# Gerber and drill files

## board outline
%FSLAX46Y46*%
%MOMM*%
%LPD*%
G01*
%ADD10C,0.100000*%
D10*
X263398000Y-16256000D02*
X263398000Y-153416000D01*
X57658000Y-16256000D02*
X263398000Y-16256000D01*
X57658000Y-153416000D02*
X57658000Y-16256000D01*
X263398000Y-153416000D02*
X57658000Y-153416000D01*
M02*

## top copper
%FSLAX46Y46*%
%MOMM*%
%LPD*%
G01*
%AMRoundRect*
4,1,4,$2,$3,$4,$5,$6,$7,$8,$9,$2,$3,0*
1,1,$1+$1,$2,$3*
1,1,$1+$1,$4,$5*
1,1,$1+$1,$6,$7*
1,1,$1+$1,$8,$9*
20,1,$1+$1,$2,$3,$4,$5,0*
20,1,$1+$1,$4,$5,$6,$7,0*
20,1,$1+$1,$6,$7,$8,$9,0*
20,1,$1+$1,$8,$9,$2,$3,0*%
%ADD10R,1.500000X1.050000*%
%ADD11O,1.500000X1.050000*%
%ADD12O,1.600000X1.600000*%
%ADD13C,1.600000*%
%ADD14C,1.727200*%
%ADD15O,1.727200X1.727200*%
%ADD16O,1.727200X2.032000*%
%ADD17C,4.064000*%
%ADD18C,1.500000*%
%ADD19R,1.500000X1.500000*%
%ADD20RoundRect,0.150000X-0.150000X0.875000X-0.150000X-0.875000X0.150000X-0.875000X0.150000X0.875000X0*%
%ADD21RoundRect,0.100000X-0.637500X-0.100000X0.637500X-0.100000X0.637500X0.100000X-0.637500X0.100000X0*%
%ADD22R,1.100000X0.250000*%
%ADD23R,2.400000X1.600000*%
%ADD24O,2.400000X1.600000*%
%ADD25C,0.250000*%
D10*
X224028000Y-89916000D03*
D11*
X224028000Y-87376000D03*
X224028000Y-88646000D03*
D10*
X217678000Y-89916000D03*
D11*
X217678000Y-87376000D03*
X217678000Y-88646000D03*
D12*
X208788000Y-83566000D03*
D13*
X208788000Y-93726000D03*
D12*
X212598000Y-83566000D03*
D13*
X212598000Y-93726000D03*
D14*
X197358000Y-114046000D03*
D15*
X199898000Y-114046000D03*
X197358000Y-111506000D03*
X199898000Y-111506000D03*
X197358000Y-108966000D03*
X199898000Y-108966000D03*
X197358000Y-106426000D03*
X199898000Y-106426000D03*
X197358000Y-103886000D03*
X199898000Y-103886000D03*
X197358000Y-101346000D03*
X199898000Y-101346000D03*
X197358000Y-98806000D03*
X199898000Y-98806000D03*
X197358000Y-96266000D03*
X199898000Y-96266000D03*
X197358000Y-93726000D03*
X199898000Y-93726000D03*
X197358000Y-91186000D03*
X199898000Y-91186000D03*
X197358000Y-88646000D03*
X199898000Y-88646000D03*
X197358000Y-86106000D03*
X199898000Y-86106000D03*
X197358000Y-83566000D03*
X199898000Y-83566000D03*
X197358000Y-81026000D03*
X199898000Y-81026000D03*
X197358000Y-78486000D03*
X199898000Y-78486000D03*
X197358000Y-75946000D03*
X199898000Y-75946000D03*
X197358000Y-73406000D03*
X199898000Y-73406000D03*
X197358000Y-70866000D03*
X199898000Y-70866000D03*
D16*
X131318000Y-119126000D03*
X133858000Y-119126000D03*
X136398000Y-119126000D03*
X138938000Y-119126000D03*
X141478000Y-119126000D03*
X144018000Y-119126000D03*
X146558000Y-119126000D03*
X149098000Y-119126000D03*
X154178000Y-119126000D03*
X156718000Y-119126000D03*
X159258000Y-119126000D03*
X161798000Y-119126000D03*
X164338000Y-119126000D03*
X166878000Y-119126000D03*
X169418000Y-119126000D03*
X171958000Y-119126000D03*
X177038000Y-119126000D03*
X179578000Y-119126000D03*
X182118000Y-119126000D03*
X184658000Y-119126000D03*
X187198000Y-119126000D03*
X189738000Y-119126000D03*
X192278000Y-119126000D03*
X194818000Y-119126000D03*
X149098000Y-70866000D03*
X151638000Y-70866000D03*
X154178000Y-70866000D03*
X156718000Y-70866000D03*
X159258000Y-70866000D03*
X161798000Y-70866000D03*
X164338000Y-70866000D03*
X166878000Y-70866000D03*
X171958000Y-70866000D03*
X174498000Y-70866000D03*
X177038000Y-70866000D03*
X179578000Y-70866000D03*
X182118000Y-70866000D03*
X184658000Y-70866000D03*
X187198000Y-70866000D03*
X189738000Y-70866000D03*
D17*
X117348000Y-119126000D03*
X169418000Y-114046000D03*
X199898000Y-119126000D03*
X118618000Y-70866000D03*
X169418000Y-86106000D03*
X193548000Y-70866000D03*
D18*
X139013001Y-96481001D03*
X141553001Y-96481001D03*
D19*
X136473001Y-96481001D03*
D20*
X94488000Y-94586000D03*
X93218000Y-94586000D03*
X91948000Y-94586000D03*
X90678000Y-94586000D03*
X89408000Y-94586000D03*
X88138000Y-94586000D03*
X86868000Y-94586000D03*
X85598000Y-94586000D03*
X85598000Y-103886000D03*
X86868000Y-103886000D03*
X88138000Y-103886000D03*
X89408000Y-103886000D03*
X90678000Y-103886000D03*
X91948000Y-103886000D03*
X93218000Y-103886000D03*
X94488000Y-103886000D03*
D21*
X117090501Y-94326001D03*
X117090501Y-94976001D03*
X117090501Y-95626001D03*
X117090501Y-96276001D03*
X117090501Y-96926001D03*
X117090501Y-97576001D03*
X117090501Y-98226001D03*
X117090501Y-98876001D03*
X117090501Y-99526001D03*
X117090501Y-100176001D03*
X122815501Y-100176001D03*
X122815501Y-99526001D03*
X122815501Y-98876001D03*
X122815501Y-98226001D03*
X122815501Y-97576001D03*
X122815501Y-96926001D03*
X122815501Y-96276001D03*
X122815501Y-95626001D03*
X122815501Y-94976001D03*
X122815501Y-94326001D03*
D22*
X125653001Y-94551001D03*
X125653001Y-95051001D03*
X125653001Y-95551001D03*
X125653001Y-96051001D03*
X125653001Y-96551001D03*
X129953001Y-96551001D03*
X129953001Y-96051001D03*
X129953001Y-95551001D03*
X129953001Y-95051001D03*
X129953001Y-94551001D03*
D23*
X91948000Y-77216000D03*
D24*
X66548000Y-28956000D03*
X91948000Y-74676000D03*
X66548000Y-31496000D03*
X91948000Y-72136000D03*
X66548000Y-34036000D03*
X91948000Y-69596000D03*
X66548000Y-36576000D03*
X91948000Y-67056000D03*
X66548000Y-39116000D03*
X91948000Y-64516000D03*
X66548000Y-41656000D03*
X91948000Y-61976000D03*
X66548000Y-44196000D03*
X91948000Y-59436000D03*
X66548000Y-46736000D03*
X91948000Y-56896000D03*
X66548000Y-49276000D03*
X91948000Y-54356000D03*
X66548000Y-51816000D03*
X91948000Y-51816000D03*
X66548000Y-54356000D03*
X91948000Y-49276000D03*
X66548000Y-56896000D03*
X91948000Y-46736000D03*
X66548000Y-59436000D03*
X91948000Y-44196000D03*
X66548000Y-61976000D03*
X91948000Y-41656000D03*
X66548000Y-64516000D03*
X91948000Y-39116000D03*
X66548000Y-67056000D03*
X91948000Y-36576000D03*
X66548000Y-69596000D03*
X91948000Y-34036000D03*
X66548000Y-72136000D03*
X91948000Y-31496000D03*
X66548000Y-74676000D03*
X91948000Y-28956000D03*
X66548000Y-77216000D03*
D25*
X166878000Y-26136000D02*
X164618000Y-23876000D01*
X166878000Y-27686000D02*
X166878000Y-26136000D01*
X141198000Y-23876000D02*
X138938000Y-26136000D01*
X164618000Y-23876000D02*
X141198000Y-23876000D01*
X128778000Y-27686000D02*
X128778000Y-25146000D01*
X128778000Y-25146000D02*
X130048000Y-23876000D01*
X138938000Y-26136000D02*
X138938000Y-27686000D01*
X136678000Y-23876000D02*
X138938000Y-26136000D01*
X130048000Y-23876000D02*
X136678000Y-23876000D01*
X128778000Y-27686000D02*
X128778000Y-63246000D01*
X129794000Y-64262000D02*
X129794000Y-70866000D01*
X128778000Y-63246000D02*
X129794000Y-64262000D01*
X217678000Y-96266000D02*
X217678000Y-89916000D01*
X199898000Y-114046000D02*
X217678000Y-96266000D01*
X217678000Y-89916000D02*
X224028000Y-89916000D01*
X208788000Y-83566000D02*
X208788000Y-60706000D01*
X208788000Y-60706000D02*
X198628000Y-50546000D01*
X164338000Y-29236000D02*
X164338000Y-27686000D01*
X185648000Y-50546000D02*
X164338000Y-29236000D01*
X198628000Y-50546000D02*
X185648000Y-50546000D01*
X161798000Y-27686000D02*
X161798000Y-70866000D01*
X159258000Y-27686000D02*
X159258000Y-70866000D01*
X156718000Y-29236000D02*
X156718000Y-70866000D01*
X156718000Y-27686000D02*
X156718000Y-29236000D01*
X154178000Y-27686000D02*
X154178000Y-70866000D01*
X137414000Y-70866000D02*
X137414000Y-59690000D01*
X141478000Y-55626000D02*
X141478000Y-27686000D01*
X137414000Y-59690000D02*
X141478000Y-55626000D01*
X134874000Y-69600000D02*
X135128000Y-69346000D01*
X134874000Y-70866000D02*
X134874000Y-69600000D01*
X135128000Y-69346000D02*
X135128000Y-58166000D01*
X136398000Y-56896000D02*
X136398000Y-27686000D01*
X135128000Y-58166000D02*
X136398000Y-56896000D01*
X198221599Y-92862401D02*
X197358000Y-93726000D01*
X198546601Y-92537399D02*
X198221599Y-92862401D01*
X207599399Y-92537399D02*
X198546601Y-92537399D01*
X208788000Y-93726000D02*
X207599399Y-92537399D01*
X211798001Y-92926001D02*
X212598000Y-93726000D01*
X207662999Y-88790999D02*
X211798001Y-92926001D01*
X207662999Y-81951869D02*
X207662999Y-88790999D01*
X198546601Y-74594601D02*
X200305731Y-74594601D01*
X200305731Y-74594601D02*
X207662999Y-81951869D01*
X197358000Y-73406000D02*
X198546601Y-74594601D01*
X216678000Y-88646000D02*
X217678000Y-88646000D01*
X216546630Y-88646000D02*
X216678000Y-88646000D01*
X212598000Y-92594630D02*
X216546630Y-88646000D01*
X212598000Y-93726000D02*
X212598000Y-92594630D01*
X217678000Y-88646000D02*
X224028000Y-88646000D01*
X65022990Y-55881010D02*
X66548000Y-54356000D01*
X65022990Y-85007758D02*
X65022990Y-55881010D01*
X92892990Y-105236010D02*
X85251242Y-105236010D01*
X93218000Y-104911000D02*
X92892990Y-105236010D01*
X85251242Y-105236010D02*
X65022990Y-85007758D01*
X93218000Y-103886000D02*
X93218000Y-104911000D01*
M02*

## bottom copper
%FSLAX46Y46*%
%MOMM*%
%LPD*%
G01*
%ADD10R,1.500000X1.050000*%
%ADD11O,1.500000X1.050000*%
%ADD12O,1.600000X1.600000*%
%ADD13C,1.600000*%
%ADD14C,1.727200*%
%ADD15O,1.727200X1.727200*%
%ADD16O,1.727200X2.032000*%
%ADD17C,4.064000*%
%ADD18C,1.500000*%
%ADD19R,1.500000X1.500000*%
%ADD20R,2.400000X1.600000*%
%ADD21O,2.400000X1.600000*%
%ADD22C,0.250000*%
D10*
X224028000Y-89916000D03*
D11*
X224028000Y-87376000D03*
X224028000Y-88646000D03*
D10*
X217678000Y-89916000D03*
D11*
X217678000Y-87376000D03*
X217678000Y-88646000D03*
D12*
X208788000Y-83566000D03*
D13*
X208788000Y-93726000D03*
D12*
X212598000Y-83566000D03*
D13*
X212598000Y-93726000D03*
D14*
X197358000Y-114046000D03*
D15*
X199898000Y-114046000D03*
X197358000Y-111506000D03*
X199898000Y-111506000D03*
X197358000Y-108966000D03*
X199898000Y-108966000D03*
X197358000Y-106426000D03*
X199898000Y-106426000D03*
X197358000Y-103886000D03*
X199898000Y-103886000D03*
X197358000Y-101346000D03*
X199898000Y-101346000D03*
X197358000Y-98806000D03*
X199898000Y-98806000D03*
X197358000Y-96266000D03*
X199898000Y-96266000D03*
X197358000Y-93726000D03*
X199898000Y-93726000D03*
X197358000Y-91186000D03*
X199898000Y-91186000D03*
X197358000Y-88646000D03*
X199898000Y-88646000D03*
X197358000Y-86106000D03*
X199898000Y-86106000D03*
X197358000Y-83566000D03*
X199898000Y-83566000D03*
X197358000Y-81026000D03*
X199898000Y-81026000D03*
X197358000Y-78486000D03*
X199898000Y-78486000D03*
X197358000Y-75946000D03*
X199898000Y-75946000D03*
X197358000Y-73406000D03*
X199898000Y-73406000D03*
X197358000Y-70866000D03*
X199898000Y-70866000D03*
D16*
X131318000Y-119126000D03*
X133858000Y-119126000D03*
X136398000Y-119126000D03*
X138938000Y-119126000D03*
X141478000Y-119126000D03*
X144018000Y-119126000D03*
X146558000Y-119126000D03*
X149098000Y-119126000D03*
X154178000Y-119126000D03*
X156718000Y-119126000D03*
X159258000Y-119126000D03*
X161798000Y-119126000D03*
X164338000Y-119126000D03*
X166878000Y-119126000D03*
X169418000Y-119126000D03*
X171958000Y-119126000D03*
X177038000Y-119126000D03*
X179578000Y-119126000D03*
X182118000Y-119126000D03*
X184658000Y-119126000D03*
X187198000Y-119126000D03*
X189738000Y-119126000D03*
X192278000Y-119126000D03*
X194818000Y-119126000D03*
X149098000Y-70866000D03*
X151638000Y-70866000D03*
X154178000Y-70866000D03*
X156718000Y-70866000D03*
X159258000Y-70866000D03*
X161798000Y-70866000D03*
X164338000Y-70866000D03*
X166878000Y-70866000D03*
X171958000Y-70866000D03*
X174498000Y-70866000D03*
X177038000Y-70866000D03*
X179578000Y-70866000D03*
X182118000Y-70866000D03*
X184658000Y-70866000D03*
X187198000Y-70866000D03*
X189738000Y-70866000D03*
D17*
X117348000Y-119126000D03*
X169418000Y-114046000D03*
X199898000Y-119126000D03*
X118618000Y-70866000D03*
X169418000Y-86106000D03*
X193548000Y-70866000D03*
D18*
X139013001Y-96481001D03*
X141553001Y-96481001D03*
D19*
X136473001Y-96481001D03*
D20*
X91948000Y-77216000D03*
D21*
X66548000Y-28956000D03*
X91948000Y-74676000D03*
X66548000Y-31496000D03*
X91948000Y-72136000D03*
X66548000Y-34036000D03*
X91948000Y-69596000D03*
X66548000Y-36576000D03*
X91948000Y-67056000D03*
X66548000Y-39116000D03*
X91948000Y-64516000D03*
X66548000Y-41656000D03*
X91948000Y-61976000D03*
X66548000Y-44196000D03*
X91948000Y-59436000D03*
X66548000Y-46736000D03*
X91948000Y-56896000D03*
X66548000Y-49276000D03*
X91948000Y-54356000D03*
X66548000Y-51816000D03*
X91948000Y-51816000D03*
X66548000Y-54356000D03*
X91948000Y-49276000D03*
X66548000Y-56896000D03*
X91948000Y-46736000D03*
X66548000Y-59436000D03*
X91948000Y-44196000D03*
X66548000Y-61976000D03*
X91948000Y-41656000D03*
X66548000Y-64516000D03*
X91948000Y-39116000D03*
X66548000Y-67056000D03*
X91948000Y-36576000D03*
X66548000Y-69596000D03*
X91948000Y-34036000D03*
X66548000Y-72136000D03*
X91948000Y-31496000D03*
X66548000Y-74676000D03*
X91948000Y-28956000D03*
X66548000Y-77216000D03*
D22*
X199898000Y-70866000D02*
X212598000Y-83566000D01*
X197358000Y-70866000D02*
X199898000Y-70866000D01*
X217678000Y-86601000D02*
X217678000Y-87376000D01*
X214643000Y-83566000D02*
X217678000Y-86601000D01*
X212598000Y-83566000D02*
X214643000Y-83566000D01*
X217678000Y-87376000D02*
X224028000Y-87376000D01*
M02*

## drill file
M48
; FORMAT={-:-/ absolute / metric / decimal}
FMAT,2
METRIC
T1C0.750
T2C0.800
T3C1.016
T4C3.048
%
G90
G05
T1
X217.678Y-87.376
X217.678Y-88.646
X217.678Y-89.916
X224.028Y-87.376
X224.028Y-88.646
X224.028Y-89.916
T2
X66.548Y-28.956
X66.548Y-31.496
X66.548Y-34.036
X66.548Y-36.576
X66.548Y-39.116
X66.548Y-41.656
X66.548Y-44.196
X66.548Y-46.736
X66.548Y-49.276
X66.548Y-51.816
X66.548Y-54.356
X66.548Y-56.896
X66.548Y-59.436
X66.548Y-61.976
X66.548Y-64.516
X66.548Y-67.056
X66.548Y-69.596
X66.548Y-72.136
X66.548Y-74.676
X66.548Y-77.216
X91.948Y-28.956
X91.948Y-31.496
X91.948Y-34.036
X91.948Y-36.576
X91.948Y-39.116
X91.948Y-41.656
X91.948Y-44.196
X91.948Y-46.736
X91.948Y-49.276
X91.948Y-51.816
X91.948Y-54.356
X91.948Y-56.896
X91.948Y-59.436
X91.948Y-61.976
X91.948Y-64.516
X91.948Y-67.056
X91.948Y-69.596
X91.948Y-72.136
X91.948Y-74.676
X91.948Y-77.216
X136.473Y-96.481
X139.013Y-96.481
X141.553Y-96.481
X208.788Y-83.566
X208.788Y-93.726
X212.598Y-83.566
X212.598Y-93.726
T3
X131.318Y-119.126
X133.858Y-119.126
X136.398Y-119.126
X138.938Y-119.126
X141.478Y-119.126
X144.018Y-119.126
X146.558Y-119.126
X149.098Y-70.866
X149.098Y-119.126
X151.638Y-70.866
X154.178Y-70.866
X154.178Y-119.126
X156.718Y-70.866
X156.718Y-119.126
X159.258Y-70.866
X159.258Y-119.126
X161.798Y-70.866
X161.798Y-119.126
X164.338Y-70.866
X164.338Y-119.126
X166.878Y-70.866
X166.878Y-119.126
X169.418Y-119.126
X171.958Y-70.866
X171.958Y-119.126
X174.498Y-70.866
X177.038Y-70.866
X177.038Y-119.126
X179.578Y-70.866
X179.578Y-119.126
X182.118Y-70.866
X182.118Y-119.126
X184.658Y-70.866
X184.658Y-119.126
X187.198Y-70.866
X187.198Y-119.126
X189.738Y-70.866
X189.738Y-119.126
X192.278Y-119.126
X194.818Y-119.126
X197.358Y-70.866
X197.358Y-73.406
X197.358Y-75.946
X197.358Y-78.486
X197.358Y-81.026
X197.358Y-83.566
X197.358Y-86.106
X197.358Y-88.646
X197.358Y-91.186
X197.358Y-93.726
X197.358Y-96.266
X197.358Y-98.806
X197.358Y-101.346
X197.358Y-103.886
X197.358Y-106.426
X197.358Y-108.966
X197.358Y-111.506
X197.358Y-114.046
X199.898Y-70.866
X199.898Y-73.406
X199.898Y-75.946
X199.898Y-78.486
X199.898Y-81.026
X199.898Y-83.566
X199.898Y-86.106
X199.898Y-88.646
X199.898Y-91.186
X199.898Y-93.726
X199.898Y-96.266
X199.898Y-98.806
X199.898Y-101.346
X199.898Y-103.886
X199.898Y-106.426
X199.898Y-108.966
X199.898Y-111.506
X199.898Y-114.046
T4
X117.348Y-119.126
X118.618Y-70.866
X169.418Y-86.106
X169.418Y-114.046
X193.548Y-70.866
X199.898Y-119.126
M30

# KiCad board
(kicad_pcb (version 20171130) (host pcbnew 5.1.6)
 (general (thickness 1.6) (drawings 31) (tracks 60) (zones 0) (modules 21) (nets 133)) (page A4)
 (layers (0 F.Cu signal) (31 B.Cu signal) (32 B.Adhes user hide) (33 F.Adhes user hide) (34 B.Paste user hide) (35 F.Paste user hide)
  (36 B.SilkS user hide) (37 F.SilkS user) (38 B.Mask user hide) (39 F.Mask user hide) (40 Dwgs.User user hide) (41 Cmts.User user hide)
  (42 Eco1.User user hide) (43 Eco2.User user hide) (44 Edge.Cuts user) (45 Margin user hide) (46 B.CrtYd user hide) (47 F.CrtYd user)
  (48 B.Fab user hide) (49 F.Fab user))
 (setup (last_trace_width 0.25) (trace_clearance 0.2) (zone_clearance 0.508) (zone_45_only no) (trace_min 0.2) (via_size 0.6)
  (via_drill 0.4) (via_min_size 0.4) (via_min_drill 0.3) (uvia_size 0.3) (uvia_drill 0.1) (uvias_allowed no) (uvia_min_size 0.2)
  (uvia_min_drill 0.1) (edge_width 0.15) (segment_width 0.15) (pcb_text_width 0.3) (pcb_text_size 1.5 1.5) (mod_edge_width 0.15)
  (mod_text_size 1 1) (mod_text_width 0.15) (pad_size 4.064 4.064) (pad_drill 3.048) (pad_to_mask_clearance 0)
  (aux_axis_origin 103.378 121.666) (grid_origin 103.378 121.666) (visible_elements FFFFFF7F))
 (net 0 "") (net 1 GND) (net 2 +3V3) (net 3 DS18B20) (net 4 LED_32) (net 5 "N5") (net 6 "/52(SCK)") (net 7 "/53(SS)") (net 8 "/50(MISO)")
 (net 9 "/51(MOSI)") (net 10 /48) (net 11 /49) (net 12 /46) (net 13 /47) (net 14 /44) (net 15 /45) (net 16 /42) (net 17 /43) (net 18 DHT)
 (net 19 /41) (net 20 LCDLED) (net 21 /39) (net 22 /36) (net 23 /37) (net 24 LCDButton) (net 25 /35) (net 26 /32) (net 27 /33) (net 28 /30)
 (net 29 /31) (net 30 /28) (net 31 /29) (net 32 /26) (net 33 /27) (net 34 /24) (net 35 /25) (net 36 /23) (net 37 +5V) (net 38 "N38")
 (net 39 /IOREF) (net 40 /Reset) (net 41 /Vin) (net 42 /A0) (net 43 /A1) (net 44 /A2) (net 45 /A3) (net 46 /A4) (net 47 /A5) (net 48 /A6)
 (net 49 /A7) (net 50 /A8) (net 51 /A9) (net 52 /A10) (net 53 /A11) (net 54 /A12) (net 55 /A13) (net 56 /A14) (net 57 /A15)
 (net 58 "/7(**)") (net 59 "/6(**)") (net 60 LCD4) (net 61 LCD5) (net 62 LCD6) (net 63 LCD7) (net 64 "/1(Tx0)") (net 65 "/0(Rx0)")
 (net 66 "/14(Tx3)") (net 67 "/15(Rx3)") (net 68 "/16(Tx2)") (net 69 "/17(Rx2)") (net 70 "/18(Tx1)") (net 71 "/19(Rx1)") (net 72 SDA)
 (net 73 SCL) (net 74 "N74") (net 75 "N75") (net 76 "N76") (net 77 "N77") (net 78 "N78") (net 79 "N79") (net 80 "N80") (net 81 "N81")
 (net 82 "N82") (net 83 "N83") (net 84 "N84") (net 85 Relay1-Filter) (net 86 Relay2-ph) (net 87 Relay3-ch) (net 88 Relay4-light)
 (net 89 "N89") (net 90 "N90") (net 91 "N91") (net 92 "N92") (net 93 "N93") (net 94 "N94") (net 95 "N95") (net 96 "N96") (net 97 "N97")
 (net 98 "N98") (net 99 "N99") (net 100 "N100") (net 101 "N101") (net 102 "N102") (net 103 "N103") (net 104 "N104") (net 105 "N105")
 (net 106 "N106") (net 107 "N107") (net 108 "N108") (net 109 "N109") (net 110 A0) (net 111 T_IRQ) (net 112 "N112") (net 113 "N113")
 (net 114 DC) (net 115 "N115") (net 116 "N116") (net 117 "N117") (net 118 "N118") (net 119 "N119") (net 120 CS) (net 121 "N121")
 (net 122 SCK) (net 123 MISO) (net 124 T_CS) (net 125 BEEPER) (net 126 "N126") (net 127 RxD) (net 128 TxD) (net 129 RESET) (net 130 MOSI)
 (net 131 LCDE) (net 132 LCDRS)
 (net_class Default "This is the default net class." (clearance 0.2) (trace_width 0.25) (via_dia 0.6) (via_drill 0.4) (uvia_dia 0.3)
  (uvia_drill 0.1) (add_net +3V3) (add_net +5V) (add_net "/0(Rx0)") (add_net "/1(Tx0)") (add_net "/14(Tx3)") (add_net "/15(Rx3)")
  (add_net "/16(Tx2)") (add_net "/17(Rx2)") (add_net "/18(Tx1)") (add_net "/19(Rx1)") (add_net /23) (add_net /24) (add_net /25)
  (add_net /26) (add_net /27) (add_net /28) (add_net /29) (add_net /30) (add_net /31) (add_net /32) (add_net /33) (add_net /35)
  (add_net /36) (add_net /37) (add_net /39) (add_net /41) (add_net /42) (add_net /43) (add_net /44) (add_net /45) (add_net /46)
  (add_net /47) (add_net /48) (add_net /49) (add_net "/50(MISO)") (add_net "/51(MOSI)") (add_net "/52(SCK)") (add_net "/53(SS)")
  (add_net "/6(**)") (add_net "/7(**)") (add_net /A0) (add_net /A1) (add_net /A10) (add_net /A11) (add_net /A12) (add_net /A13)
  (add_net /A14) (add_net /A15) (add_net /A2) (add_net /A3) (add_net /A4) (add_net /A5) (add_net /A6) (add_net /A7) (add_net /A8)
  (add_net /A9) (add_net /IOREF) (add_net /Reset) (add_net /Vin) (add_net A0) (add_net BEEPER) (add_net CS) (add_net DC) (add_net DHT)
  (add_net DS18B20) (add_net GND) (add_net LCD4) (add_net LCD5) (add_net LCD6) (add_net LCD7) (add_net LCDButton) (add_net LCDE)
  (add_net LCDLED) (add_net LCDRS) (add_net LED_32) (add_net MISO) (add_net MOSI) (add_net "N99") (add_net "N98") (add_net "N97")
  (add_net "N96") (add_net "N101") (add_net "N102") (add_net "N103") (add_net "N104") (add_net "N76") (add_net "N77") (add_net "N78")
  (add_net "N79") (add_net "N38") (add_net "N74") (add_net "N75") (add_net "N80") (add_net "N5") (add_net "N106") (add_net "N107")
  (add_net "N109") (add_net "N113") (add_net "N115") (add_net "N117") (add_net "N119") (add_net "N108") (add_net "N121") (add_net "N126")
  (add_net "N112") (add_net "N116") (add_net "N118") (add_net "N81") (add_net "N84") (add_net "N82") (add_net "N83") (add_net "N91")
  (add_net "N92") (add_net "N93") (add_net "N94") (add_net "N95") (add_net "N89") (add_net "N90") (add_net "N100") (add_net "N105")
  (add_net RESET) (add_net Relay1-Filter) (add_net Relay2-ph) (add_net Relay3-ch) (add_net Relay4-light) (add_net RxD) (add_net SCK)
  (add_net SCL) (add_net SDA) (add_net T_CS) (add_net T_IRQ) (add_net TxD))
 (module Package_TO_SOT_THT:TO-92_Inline (layer F.Cu) (at 224.028 89.916 90)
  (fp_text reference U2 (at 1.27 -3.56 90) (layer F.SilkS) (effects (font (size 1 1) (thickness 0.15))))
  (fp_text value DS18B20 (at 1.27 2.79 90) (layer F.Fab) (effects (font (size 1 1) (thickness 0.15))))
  (pad 1 thru_hole rect (at 0 0 90) (size 1.05 1.5) (drill 0.75) (layers *.Cu *.Mask) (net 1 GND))
  (pad 3 thru_hole oval (at 2.54 0 90) (size 1.05 1.5) (drill 0.75) (layers *.Cu *.Mask) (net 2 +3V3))
  (pad 2 thru_hole oval (at 1.27 0 90) (size 1.05 1.5) (drill 0.75) (layers *.Cu *.Mask) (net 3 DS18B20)))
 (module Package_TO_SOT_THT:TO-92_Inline (layer F.Cu) (at 217.678 89.916 90)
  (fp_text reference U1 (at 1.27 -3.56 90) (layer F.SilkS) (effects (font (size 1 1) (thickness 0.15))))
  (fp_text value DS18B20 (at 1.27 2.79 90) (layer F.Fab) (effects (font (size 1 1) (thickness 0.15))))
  (pad 1 thru_hole rect (at 0 0 90) (size 1.05 1.5) (drill 0.75) (layers *.Cu *.Mask) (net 1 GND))
  (pad 3 thru_hole oval (at 2.54 0 90) (size 1.05 1.5) (drill 0.75) (layers *.Cu *.Mask) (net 2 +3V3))
  (pad 2 thru_hole oval (at 1.27 0 90) (size 1.05 1.5) (drill 0.75) (layers *.Cu *.Mask) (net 3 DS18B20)))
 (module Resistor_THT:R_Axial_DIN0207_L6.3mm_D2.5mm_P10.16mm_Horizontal (layer F.Cu) (at 208.788 93.726 90)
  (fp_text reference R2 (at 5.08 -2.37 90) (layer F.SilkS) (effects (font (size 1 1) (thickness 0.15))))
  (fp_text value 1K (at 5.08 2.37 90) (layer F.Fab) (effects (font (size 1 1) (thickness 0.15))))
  (pad 2 thru_hole oval (at 10.16 0 90) (size 1.6 1.6) (drill 0.8) (layers *.Cu *.Mask) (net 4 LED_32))
  (pad 1 thru_hole circle (at 0 0 90) (size 1.6 1.6) (drill 0.8) (layers *.Cu *.Mask) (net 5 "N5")))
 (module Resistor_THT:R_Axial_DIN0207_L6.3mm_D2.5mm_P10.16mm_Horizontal (layer F.Cu) (at 212.598 93.726 90)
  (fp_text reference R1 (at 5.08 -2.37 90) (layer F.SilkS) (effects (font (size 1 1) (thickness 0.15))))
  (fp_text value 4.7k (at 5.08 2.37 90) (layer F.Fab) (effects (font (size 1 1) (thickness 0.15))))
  (pad 2 thru_hole oval (at 10.16 0 90) (size 1.6 1.6) (drill 0.8) (layers *.Cu *.Mask) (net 2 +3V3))
  (pad 1 thru_hole circle (at 0 0 90) (size 1.6 1.6) (drill 0.8) (layers *.Cu *.Mask) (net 3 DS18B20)))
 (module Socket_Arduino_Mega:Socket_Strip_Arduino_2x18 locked (layer F.Cu) (at 197.358 114.046 90)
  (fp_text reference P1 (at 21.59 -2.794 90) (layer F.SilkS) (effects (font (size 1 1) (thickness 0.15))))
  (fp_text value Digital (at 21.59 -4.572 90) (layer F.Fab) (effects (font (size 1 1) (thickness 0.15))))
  (pad 1 thru_hole circle (at 0 0 90) (size 1.7272 1.7272) (drill 1.016) (layers *.Cu *.Mask F.SilkS) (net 1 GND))
  (pad 2 thru_hole oval (at 0 2.54 90) (size 1.7272 1.7272) (drill 1.016) (layers *.Cu *.Mask F.SilkS) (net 1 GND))
  (pad 3 thru_hole oval (at 2.54 0 90) (size 1.7272 1.7272) (drill 1.016) (layers *.Cu *.Mask F.SilkS) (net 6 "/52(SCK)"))
  (pad 4 thru_hole oval (at 2.54 2.54 90) (size 1.7272 1.7272) (drill 1.016) (layers *.Cu *.Mask F.SilkS) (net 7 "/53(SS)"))
  (pad 5 thru_hole oval (at 5.08 0 90) (size 1.7272 1.7272) (drill 1.016) (layers *.Cu *.Mask F.SilkS) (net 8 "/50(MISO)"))
  (pad 6 thru_hole oval (at 5.08 2.54 90) (size 1.7272 1.7272) (drill 1.016) (layers *.Cu *.Mask F.SilkS) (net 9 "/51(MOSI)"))
  (pad 7 thru_hole oval (at 7.62 0 90) (size 1.7272 1.7272) (drill 1.016) (layers *.Cu *.Mask F.SilkS) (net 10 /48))
  (pad 8 thru_hole oval (at 7.62 2.54 90) (size 1.7272 1.7272) (drill 1.016) (layers *.Cu *.Mask F.SilkS) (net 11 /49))
  (pad 9 thru_hole oval (at 10.16 0 90) (size 1.7272 1.7272) (drill 1.016) (layers *.Cu *.Mask F.SilkS) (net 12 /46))
  (pad 10 thru_hole oval (at 10.16 2.54 90) (size 1.7272 1.7272) (drill 1.016) (layers *.Cu *.Mask F.SilkS) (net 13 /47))
  (pad 11 thru_hole oval (at 12.7 0 90) (size 1.7272 1.7272) (drill 1.016) (layers *.Cu *.Mask F.SilkS) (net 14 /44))
  (pad 12 thru_hole oval (at 12.7 2.54 90) (size 1.7272 1.7272) (drill 1.016) (layers *.Cu *.Mask F.SilkS) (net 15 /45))
  (pad 13 thru_hole oval (at 15.24 0 90) (size 1.7272 1.7272) (drill 1.016) (layers *.Cu *.Mask F.SilkS) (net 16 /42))
  (pad 14 thru_hole oval (at 15.24 2.54 90) (size 1.7272 1.7272) (drill 1.016) (layers *.Cu *.Mask F.SilkS) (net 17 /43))
  (pad 15 thru_hole oval (at 17.78 0 90) (size 1.7272 1.7272) (drill 1.016) (layers *.Cu *.Mask F.SilkS) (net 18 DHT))
  (pad 16 thru_hole oval (at 17.78 2.54 90) (size 1.7272 1.7272) (drill 1.016) (layers *.Cu *.Mask F.SilkS) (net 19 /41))
  (pad 17 thru_hole oval (at 20.32 0 90) (size 1.7272 1.7272) (drill 1.016) (layers *.Cu *.Mask F.SilkS) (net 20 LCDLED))
  (pad 18 thru_hole oval (at 20.32 2.54 90) (size 1.7272 1.7272) (drill 1.016) (layers *.Cu *.Mask F.SilkS) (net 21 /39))
  (pad 19 thru_hole oval (at 22.86 0 90) (size 1.7272 1.7272) (drill 1.016) (layers *.Cu *.Mask F.SilkS) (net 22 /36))
  (pad 20 thru_hole oval (at 22.86 2.54 90) (size 1.7272 1.7272) (drill 1.016) (layers *.Cu *.Mask F.SilkS) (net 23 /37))
  (pad 21 thru_hole oval (at 25.4 0 90) (size 1.7272 1.7272) (drill 1.016) (layers *.Cu *.Mask F.SilkS) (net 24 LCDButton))
  (pad 22 thru_hole oval (at 25.4 2.54 90) (size 1.7272 1.7272) (drill 1.016) (layers *.Cu *.Mask F.SilkS) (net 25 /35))
  (pad 23 thru_hole oval (at 27.94 0 90) (size 1.7272 1.7272) (drill 1.016) (layers *.Cu *.Mask F.SilkS) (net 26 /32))
  (pad 24 thru_hole oval (at 27.94 2.54 90) (size 1.7272 1.7272) (drill 1.016) (layers *.Cu *.Mask F.SilkS) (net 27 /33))
  (pad 25 thru_hole oval (at 30.48 0 90) (size 1.7272 1.7272) (drill 1.016) (layers *.Cu *.Mask F.SilkS) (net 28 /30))
  (pad 26 thru_hole oval (at 30.48 2.54 90) (size 1.7272 1.7272) (drill 1.016) (layers *.Cu *.Mask F.SilkS) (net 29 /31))
  (pad 27 thru_hole oval (at 33.02 0 90) (size 1.7272 1.7272) (drill 1.016) (layers *.Cu *.Mask F.SilkS) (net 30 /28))
  (pad 28 thru_hole oval (at 33.02 2.54 90) (size 1.7272 1.7272) (drill 1.016) (layers *.Cu *.Mask F.SilkS) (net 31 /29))
  (pad 29 thru_hole oval (at 35.56 0 90) (size 1.7272 1.7272) (drill 1.016) (layers *.Cu *.Mask F.SilkS) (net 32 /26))
  (pad 30 thru_hole oval (at 35.56 2.54 90) (size 1.7272 1.7272) (drill 1.016) (layers *.Cu *.Mask F.SilkS) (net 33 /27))
  (pad 31 thru_hole oval (at 38.1 0 90) (size 1.7272 1.7272) (drill 1.016) (layers *.Cu *.Mask F.SilkS) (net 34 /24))
  (pad 32 thru_hole oval (at 38.1 2.54 90) (size 1.7272 1.7272) (drill 1.016) (layers *.Cu *.Mask F.SilkS) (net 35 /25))
  (pad 33 thru_hole oval (at 40.64 0 90) (size 1.7272 1.7272) (drill 1.016) (layers *.Cu *.Mask F.SilkS) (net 3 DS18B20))
  (pad 34 thru_hole oval (at 40.64 2.54 90) (size 1.7272 1.7272) (drill 1.016) (layers *.Cu *.Mask F.SilkS) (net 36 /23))
  (pad 35 thru_hole oval (at 43.18 0 90) (size 1.7272 1.7272) (drill 1.016) (layers *.Cu *.Mask F.SilkS) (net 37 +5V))
  (pad 36 thru_hole oval (at 43.18 2.54 90) (size 1.7272 1.7272) (drill 1.016) (layers *.Cu *.Mask F.SilkS) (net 37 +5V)))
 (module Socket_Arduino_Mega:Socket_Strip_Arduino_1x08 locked (layer F.Cu) (at 131.318 119.126)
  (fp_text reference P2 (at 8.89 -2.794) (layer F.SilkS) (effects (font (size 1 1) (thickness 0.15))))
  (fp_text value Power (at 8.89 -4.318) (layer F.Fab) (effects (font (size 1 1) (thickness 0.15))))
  (pad 1 thru_hole oval (at 0 0) (size 1.7272 2.032) (drill 1.016) (layers *.Cu *.Mask F.SilkS) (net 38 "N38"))
  (pad 2 thru_hole oval (at 2.54 0) (size 1.7272 2.032) (drill 1.016) (layers *.Cu *.Mask F.SilkS) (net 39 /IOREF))
  (pad 3 thru_hole oval (at 5.08 0) (size 1.7272 2.032) (drill 1.016) (layers *.Cu *.Mask F.SilkS) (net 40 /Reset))
  (pad 4 thru_hole oval (at 7.62 0) (size 1.7272 2.032) (drill 1.016) (layers *.Cu *.Mask F.SilkS) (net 2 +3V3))
  (pad 5 thru_hole oval (at 10.16 0) (size 1.7272 2.032) (drill 1.016) (layers *.Cu *.Mask F.SilkS) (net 37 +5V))
  (pad 6 thru_hole oval (at 12.7 0) (size 1.7272 2.032) (drill 1.016) (layers *.Cu *.Mask F.SilkS) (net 1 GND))
  (pad 7 thru_hole oval (at 15.24 0) (size 1.7272 2.032) (drill 1.016) (layers *.Cu *.Mask F.SilkS) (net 1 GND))
  (pad 8 thru_hole oval (at 17.78 0) (size 1.7272 2.032) (drill 1.016) (layers *.Cu *.Mask F.SilkS) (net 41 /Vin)))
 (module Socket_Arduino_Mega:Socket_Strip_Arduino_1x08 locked (layer F.Cu) (at 154.178 119.126)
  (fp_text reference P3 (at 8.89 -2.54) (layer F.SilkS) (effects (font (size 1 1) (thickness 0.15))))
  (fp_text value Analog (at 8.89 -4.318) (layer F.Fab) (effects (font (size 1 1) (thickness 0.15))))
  (pad 1 thru_hole oval (at 0 0) (size 1.7272 2.032) (drill 1.016) (layers *.Cu *.Mask F.SilkS) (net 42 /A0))
  (pad 2 thru_hole oval (at 2.54 0) (size 1.7272 2.032) (drill 1.016) (layers *.Cu *.Mask F.SilkS) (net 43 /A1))
  (pad 3 thru_hole oval (at 5.08 0) (size 1.7272 2.032) (drill 1.016) (layers *.Cu *.Mask F.SilkS) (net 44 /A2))
  (pad 4 thru_hole oval (at 7.62 0) (size 1.7272 2.032) (drill 1.016) (layers *.Cu *.Mask F.SilkS) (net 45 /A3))
  (pad 5 thru_hole oval (at 10.16 0) (size 1.7272 2.032) (drill 1.016) (layers *.Cu *.Mask F.SilkS) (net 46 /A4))
  (pad 6 thru_hole oval (at 12.7 0) (size 1.7272 2.032) (drill 1.016) (layers *.Cu *.Mask F.SilkS) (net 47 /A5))
  (pad 7 thru_hole oval (at 15.24 0) (size 1.7272 2.032) (drill 1.016) (layers *.Cu *.Mask F.SilkS) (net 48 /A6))
  (pad 8 thru_hole oval (at 17.78 0) (size 1.7272 2.032) (drill 1.016) (layers *.Cu *.Mask F.SilkS) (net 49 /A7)))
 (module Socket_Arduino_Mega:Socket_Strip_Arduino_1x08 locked (layer F.Cu) (at 177.038 119.126)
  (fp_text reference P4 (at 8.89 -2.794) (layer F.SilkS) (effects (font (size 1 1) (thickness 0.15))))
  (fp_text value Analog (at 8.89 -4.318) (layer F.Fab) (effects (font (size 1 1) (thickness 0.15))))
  (pad 1 thru_hole oval (at 0 0) (size 1.7272 2.032) (drill 1.016) (layers *.Cu *.Mask F.SilkS) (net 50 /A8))
  (pad 2 thru_hole oval (at 2.54 0) (size 1.7272 2.032) (drill 1.016) (layers *.Cu *.Mask F.SilkS) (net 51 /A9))
  (pad 3 thru_hole oval (at 5.08 0) (size 1.7272 2.032) (drill 1.016) (layers *.Cu *.Mask F.SilkS) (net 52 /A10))
  (pad 4 thru_hole oval (at 7.62 0) (size 1.7272 2.032) (drill 1.016) (layers *.Cu *.Mask F.SilkS) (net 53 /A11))
  (pad 5 thru_hole oval (at 10.16 0) (size 1.7272 2.032) (drill 1.016) (layers *.Cu *.Mask F.SilkS) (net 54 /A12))
  (pad 6 thru_hole oval (at 12.7 0) (size 1.7272 2.032) (drill 1.016) (layers *.Cu *.Mask F.SilkS) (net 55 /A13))
  (pad 7 thru_hole oval (at 15.24 0) (size 1.7272 2.032) (drill 1.016) (layers *.Cu *.Mask F.SilkS) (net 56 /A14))
  (pad 8 thru_hole oval (at 17.78 0) (size 1.7272 2.032) (drill 1.016) (layers *.Cu *.Mask F.SilkS) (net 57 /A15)))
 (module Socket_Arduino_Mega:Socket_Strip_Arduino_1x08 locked (layer F.Cu) (at 149.098 70.866)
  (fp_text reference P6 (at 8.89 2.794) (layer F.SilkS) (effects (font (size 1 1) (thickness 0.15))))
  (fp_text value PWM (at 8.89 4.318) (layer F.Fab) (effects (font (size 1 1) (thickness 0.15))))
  (pad 1 thru_hole oval (at 0 0) (size 1.7272 2.032) (drill 1.016) (layers *.Cu *.Mask F.SilkS) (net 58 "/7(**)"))
  (pad 2 thru_hole oval (at 2.54 0) (size 1.7272 2.032) (drill 1.016) (layers *.Cu *.Mask F.SilkS) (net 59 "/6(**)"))
  (pad 3 thru_hole oval (at 5.08 0) (size 1.7272 2.032) (drill 1.016) (layers *.Cu *.Mask F.SilkS) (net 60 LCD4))
  (pad 4 thru_hole oval (at 7.62 0) (size 1.7272 2.032) (drill 1.016) (layers *.Cu *.Mask F.SilkS) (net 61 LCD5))
  (pad 5 thru_hole oval (at 10.16 0) (size 1.7272 2.032) (drill 1.016) (layers *.Cu *.Mask F.SilkS) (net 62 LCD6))
  (pad 6 thru_hole oval (at 12.7 0) (size 1.7272 2.032) (drill 1.016) (layers *.Cu *.Mask F.SilkS) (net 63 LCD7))
  (pad 7 thru_hole oval (at 15.24 0) (size 1.7272 2.032) (drill 1.016) (layers *.Cu *.Mask F.SilkS) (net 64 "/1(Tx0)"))
  (pad 8 thru_hole oval (at 17.78 0) (size 1.7272 2.032) (drill 1.016) (layers *.Cu *.Mask F.SilkS) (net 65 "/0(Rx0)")))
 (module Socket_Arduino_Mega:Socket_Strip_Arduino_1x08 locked (layer F.Cu) (at 171.958 70.866)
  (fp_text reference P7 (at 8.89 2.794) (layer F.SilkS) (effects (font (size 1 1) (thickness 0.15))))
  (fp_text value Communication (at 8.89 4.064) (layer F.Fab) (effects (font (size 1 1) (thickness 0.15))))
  (pad 1 thru_hole oval (at 0 0) (size 1.7272 2.032) (drill 1.016) (layers *.Cu *.Mask F.SilkS) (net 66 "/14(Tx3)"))
  (pad 2 thru_hole oval (at 2.54 0) (size 1.7272 2.032) (drill 1.016) (layers *.Cu *.Mask F.SilkS) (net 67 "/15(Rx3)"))
  (pad 3 thru_hole oval (at 5.08 0) (size 1.7272 2.032) (drill 1.016) (layers *.Cu *.Mask F.SilkS) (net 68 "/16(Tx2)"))
  (pad 4 thru_hole oval (at 7.62 0) (size 1.7272 2.032) (drill 1.016) (layers *.Cu *.Mask F.SilkS) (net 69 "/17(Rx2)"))
  (pad 5 thru_hole oval (at 10.16 0) (size 1.7272 2.032) (drill 1.016) (layers *.Cu *.Mask F.SilkS) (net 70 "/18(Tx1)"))
  (pad 6 thru_hole oval (at 12.7 0) (size 1.7272 2.032) (drill 1.016) (layers *.Cu *.Mask F.SilkS) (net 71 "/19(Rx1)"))
  (pad 7 thru_hole oval (at 15.24 0) (size 1.7272 2.032) (drill 1.016) (layers *.Cu *.Mask F.SilkS) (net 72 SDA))
  (pad 8 thru_hole oval (at 17.78 0) (size 1.7272 2.032) (drill 1.016) (layers *.Cu *.Mask F.SilkS) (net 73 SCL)))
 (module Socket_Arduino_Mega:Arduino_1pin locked (layer F.Cu) (at 117.348 119.126)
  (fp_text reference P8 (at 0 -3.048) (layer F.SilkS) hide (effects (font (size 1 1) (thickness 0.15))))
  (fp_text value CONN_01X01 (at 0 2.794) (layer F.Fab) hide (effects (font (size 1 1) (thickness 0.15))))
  (pad 1 thru_hole circle (at 0 0) (size 4.064 4.064) (drill 3.048) (layers *.Cu *.Mask F.SilkS) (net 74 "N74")))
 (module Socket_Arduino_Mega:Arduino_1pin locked (layer F.Cu) (at 169.418 114.046)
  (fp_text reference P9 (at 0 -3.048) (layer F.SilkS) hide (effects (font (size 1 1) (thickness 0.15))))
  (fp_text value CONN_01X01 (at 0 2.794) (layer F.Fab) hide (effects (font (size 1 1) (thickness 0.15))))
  (pad 1 thru_hole circle (at 0 0) (size 4.064 4.064) (drill 3.048) (layers *.Cu *.Mask F.SilkS) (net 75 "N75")))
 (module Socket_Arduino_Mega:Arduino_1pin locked (layer F.Cu) (at 199.898 119.126)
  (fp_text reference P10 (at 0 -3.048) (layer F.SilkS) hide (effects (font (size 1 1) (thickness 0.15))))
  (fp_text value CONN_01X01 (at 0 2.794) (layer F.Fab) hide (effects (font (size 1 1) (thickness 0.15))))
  (pad 1 thru_hole circle (at 0 0) (size 4.064 4.064) (drill 3.048) (layers *.Cu *.Mask F.SilkS) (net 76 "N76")))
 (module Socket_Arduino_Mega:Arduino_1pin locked (layer F.Cu) (at 118.618 70.866)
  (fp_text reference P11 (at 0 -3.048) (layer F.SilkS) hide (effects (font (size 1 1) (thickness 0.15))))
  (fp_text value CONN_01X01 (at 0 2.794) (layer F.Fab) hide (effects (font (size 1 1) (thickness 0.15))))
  (pad 1 thru_hole circle (at 0 0) (size 4.064 4.064) (drill 3.048) (layers *.Cu *.Mask F.SilkS) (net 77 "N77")))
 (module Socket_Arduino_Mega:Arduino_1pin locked (layer F.Cu) (at 169.418 86.106)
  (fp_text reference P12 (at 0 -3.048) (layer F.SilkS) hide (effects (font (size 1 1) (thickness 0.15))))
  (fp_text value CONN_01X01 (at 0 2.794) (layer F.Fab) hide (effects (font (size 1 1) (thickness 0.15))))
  (pad 1 thru_hole circle (at 0 0) (size 4.064 4.064) (drill 3.048) (layers *.Cu *.Mask F.SilkS) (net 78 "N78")))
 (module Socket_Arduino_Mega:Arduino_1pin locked (layer F.Cu) (at 193.548 70.866)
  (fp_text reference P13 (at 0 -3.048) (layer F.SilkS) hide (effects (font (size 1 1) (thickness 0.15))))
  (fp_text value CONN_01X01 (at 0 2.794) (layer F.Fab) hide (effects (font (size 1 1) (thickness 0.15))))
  (pad 1 thru_hole circle (at 0 0) (size 4.064 4.064) (drill 3.048) (layers *.Cu *.Mask F.SilkS) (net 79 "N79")))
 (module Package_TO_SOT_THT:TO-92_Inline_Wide (layer F.Cu) (at 136.473001 96.481001)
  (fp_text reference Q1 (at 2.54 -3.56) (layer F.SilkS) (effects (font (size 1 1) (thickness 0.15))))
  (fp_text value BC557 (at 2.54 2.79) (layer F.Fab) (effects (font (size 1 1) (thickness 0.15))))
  (pad 2 thru_hole circle (at 2.54 0 90) (size 1.5 1.5) (drill 0.8) (layers *.Cu *.Mask) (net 5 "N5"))
  (pad 3 thru_hole circle (at 5.08 0 90) (size 1.5 1.5) (drill 0.8) (layers *.Cu *.Mask) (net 2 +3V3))
  (pad 1 thru_hole rect (at 0 0 90) (size 1.5 1.5) (drill 0.8) (layers *.Cu *.Mask) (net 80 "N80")))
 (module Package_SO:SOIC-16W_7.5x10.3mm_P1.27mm (layer F.Cu) (at 90.043 99.236 270)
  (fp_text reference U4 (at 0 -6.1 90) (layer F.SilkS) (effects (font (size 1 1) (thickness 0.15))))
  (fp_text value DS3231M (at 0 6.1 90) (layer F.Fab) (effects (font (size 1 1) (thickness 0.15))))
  (pad 1 smd roundrect (at -4.65 -4.445 270) (size 2.05 0.6) (layers F.Cu F.Paste F.Mask) (roundrect_rratio 0.25) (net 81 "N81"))
  (pad 2 smd roundrect (at -4.65 -3.175 270) (size 2.05 0.6) (layers F.Cu F.Paste F.Mask) (roundrect_rratio 0.25) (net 2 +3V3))
  (pad 3 smd roundrect (at -4.65 -1.905 270) (size 2.05 0.6) (layers F.Cu F.Paste F.Mask) (roundrect_rratio 0.25) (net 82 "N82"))
  (pad 4 smd roundrect (at -4.65 -0.635 270) (size 2.05 0.6) (layers F.Cu F.Paste F.Mask) (roundrect_rratio 0.25) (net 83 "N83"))
  (pad 5 smd roundrect (at -4.65 0.635 270) (size 2.05 0.6) (layers F.Cu F.Paste F.Mask) (roundrect_rratio 0.25) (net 1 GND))
  (pad 6 smd roundrect (at -4.65 1.905 270) (size 2.05 0.6) (layers F.Cu F.Paste F.Mask) (roundrect_rratio 0.25) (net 1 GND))
  (pad 7 smd roundrect (at -4.65 3.175 270) (size 2.05 0.6) (layers F.Cu F.Paste F.Mask) (roundrect_rratio 0.25) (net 1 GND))
  (pad 8 smd roundrect (at -4.65 4.445 270) (size 2.05 0.6) (layers F.Cu F.Paste F.Mask) (roundrect_rratio 0.25) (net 1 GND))
  (pad 9 smd roundrect (at 4.65 4.445 270) (size 2.05 0.6) (layers F.Cu F.Paste F.Mask) (roundrect_rratio 0.25) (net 1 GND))
  (pad 10 smd roundrect (at 4.65 3.175 270) (size 2.05 0.6) (layers F.Cu F.Paste F.Mask) (roundrect_rratio 0.25) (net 1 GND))
  (pad 11 smd roundrect (at 4.65 1.905 270) (size 2.05 0.6) (layers F.Cu F.Paste F.Mask) (roundrect_rratio 0.25) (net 1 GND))
  (pad 12 smd roundrect (at 4.65 0.635 270) (size 2.05 0.6) (layers F.Cu F.Paste F.Mask) (roundrect_rratio 0.25) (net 1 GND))
  (pad 13 smd roundrect (at 4.65 -0.635 270) (size 2.05 0.6) (layers F.Cu F.Paste F.Mask) (roundrect_rratio 0.25) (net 1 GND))
  (pad 14 smd roundrect (at 4.65 -1.905 270) (size 2.05 0.6) (layers F.Cu F.Paste F.Mask) (roundrect_rratio 0.25) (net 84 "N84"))
  (pad 15 smd roundrect (at 4.65 -3.175 270) (size 2.05 0.6) (layers F.Cu F.Paste F.Mask) (roundrect_rratio 0.25) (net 72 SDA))
  (pad 16 smd roundrect (at 4.65 -4.445 270) (size 2.05 0.6) (layers F.Cu F.Paste F.Mask) (roundrect_rratio 0.25) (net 73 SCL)))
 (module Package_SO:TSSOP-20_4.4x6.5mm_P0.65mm (layer F.Cu) (at 119.953001 97.251001)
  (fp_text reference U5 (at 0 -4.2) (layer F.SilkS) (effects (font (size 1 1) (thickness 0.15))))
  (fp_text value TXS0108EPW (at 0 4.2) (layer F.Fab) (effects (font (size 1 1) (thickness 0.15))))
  (pad 1 smd roundrect (at -2.8625 -2.925) (size 1.475 0.4) (layers F.Cu F.Paste F.Mask) (roundrect_rratio 0.25) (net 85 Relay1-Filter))
  (pad 2 smd roundrect (at -2.8625 -2.275) (size 1.475 0.4) (layers F.Cu F.Paste F.Mask) (roundrect_rratio 0.25) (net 2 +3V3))
  (pad 3 smd roundrect (at -2.8625 -1.625) (size 1.475 0.4) (layers F.Cu F.Paste F.Mask) (roundrect_rratio 0.25) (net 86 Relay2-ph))
  (pad 4 smd roundrect (at -2.8625 -0.975) (size 1.475 0.4) (layers F.Cu F.Paste F.Mask) (roundrect_rratio 0.25) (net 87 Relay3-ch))
  (pad 5 smd roundrect (at -2.8625 -0.325) (size 1.475 0.4) (layers F.Cu F.Paste F.Mask) (roundrect_rratio 0.25) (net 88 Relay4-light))
  (pad 6 smd roundrect (at -2.8625 0.325) (size 1.475 0.4) (layers F.Cu F.Paste F.Mask) (roundrect_rratio 0.25) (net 73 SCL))
  (pad 7 smd roundrect (at -2.8625 0.975) (size 1.475 0.4) (layers F.Cu F.Paste F.Mask) (roundrect_rratio 0.25) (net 72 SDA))
  (pad 8 smd roundrect (at -2.8625 1.625) (size 1.475 0.4) (layers F.Cu F.Paste F.Mask) (roundrect_rratio 0.25) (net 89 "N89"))
  (pad 9 smd roundrect (at -2.8625 2.275) (size 1.475 0.4) (layers F.Cu F.Paste F.Mask) (roundrect_rratio 0.25) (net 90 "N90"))
  (pad 10 smd roundrect (at -2.8625 2.925) (size 1.475 0.4) (layers F.Cu F.Paste F.Mask) (roundrect_rratio 0.25) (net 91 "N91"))
  (pad 11 smd roundrect (at 2.8625 2.925) (size 1.475 0.4) (layers F.Cu F.Paste F.Mask) (roundrect_rratio 0.25) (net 1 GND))
  (pad 12 smd roundrect (at 2.8625 2.275) (size 1.475 0.4) (layers F.Cu F.Paste F.Mask) (roundrect_rratio 0.25) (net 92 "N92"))
  (pad 13 smd roundrect (at 2.8625 1.625) (size 1.475 0.4) (layers F.Cu F.Paste F.Mask) (roundrect_rratio 0.25) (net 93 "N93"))
  (pad 14 smd roundrect (at 2.8625 0.975) (size 1.475 0.4) (layers F.Cu F.Paste F.Mask) (roundrect_rratio 0.25) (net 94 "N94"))
  (pad 15 smd roundrect (at 2.8625 0.325) (size 1.475 0.4) (layers F.Cu F.Paste F.Mask) (roundrect_rratio 0.25) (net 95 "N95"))
  (pad 16 smd roundrect (at 2.8625 -0.325) (size 1.475 0.4) (layers F.Cu F.Paste F.Mask) (roundrect_rratio 0.25) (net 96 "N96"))
  (pad 17 smd roundrect (at 2.8625 -0.975) (size 1.475 0.4) (layers F.Cu F.Paste F.Mask) (roundrect_rratio 0.25) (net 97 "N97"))
  (pad 18 smd roundrect (at 2.8625 -1.625) (size 1.475 0.4) (layers F.Cu F.Paste F.Mask) (roundrect_rratio 0.25) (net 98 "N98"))
  (pad 19 smd roundrect (at 2.8625 -2.275) (size 1.475 0.4) (layers F.Cu F.Paste F.Mask) (roundrect_rratio 0.25) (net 37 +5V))
  (pad 20 smd roundrect (at 2.8625 -2.925) (size 1.475 0.4) (layers F.Cu F.Paste F.Mask) (roundrect_rratio 0.25) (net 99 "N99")))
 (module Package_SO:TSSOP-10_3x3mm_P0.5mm (layer F.Cu) (at 127.803001 95.551001)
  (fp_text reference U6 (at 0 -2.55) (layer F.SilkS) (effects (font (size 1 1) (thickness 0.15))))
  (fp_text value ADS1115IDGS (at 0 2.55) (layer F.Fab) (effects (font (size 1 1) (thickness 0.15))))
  (pad 1 smd rect (at -2.15 -1) (size 1.1 0.25) (layers F.Cu F.Paste F.Mask) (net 93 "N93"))
  (pad 2 smd rect (at -2.15 -0.5) (size 1.1 0.25) (layers F.Cu F.Paste F.Mask) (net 92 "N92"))
  (pad 3 smd rect (at -2.15 0) (size 1.1 0.25) (layers F.Cu F.Paste F.Mask) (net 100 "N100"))
  (pad 4 smd rect (at -2.15 0.5) (size 1.1 0.25) (layers F.Cu F.Paste F.Mask) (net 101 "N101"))
  (pad 5 smd rect (at -2.15 1) (size 1.1 0.25) (layers F.Cu F.Paste F.Mask) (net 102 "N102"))
  (pad 6 smd rect (at 2.15 1) (size 1.1 0.25) (layers F.Cu F.Paste F.Mask) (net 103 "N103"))
  (pad 7 smd rect (at 2.15 0.5) (size 1.1 0.25) (layers F.Cu F.Paste F.Mask) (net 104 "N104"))
  (pad 8 smd rect (at 2.15 0) (size 1.1 0.25) (layers F.Cu F.Paste F.Mask) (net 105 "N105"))
  (pad 9 smd rect (at 2.15 -0.5) (size 1.1 0.25) (layers F.Cu F.Paste F.Mask) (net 94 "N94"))
  (pad 10 smd rect (at 2.15 -1) (size 1.1 0.25) (layers F.Cu F.Paste F.Mask) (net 95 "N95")))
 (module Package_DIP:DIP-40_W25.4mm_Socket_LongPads (layer F.Cu) (at 91.948 77.216 180)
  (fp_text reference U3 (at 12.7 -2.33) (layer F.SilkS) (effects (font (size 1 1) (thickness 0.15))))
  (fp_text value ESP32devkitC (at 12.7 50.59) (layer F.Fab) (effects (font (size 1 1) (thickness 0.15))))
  (pad 1 thru_hole rect (at 0 0 180) (size 2.4 1.6) (drill 0.8) (layers *.Cu *.Mask) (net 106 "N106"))
  (pad 21 thru_hole oval (at 25.4 48.26 180) (size 2.4 1.6) (drill 0.8) (layers *.Cu *.Mask))
  (pad 2 thru_hole oval (at 0 2.54 180) (size 2.4 1.6) (drill 0.8) (layers *.Cu *.Mask) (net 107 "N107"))
  (pad 22 thru_hole oval (at 25.4 45.72 180) (size 2.4 1.6) (drill 0.8) (layers *.Cu *.Mask) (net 2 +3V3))
  (pad 3 thru_hole oval (at 0 5.08 180) (size 2.4 1.6) (drill 0.8) (layers *.Cu *.Mask) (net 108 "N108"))
  (pad 23 thru_hole oval (at 25.4 43.18 180) (size 2.4 1.6) (drill 0.8) (layers *.Cu *.Mask) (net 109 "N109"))
  (pad 4 thru_hole oval (at 0 7.62 180) (size 2.4 1.6) (drill 0.8) (layers *.Cu *.Mask) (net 4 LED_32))
  (pad 24 thru_hole oval (at 25.4 40.64 180) (size 2.4 1.6) (drill 0.8) (layers *.Cu *.Mask) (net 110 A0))
  (pad 5 thru_hole oval (at 0 10.16 180) (size 2.4 1.6) (drill 0.8) (layers *.Cu *.Mask) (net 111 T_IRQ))
  (pad 25 thru_hole oval (at 25.4 38.1 180) (size 2.4 1.6) (drill 0.8) (layers *.Cu *.Mask) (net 3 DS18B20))
  (pad 6 thru_hole oval (at 0 12.7 180) (size 2.4 1.6) (drill 0.8) (layers *.Cu *.Mask) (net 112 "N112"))
  (pad 26 thru_hole oval (at 25.4 35.56 180) (size 2.4 1.6) (drill 0.8) (layers *.Cu *.Mask) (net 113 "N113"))
  (pad 7 thru_hole oval (at 0 15.24 180) (size 2.4 1.6) (drill 0.8) (layers *.Cu *.Mask) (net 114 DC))
  (pad 27 thru_hole oval (at 25.4 33.02 180) (size 2.4 1.6) (drill 0.8) (layers *.Cu *.Mask) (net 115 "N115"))
  (pad 8 thru_hole oval (at 0 17.78 180) (size 2.4 1.6) (drill 0.8) (layers *.Cu *.Mask) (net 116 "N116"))
  (pad 28 thru_hole oval (at 25.4 30.48 180) (size 2.4 1.6) (drill 0.8) (layers *.Cu *.Mask) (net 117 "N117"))
  (pad 9 thru_hole oval (at 0 20.32 180) (size 2.4 1.6) (drill 0.8) (layers *.Cu *.Mask) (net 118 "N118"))
  (pad 29 thru_hole oval (at 25.4 27.94 180) (size 2.4 1.6) (drill 0.8) (layers *.Cu *.Mask) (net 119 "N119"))
  (pad 10 thru_hole oval (at 0 22.86 180) (size 2.4 1.6) (drill 0.8) (layers *.Cu *.Mask) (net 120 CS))
  (pad 30 thru_hole oval (at 25.4 25.4 180) (size 2.4 1.6) (drill 0.8) (layers *.Cu *.Mask) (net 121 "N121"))
  (pad 11 thru_hole oval (at 0 25.4 180) (size 2.4 1.6) (drill 0.8) (layers *.Cu *.Mask) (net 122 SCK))
  (pad 31 thru_hole oval (at 25.4 22.86 180) (size 2.4 1.6) (drill 0.8) (layers *.Cu *.Mask) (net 72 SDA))
  (pad 12 thru_hole oval (at 0 27.94 180) (size 2.4 1.6) (drill 0.8) (layers *.Cu *.Mask) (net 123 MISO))
  (pad 32 thru_hole oval (at 25.4 20.32 180) (size 2.4 1.6) (drill 0.8) (layers *.Cu *.Mask) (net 73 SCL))
  (pad 13 thru_hole oval (at 0 30.48 180) (size 2.4 1.6) (drill 0.8) (layers *.Cu *.Mask) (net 1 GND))
  (pad 33 thru_hole oval (at 25.4 17.78 180) (size 2.4 1.6) (drill 0.8) (layers *.Cu *.Mask) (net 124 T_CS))
  (pad 14 thru_hole oval (at 0 33.02 180) (size 2.4 1.6) (drill 0.8) (layers *.Cu *.Mask) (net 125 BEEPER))
  (pad 34 thru_hole oval (at 25.4 15.24 180) (size 2.4 1.6) (drill 0.8) (layers *.Cu *.Mask) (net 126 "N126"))
  (pad 15 thru_hole oval (at 0 35.56 180) (size 2.4 1.6) (drill 0.8) (layers *.Cu *.Mask) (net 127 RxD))
  (pad 35 thru_hole oval (at 25.4 12.7 180) (size 2.4 1.6) (drill 0.8) (layers *.Cu *.Mask) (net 1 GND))
  (pad 16 thru_hole oval (at 0 38.1 180) (size 2.4 1.6) (drill 0.8) (layers *.Cu *.Mask) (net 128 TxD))
  (pad 36 thru_hole oval (at 25.4 10.16 180) (size 2.4 1.6) (drill 0.8) (layers *.Cu *.Mask) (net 85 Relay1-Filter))
  (pad 17 thru_hole oval (at 0 40.64 180) (size 2.4 1.6) (drill 0.8) (layers *.Cu *.Mask) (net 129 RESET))
  (pad 37 thru_hole oval (at 25.4 7.62 180) (size 2.4 1.6) (drill 0.8) (layers *.Cu *.Mask) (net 86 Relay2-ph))
  (pad 18 thru_hole oval (at 0 43.18 180) (size 2.4 1.6) (drill 0.8) (layers *.Cu *.Mask) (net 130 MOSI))
  (pad 38 thru_hole oval (at 25.4 5.08 180) (size 2.4 1.6) (drill 0.8) (layers *.Cu *.Mask) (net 87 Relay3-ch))
  (pad 19 thru_hole oval (at 0 45.72 180) (size 2.4 1.6) (drill 0.8) (layers *.Cu *.Mask) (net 1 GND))
  (pad 39 thru_hole oval (at 25.4 2.54 180) (size 2.4 1.6) (drill 0.8) (layers *.Cu *.Mask) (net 88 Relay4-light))
  (pad 20 thru_hole oval (at 0 48.26 180) (size 2.4 1.6) (drill 0.8) (layers *.Cu *.Mask))
  (pad 40 thru_hole oval (at 25.4 0 180) (size 2.4 1.6) (drill 0.8) (layers *.Cu *.Mask) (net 37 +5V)))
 (gr_line (start 263.398 16.256) (end 263.398 153.416) (layer Edge.Cuts) (width 0.1))
 (gr_line (start 57.658 16.256) (end 263.398 16.256) (layer Edge.Cuts) (width 0.1))
 (gr_line (start 57.658 153.416) (end 57.658 16.256) (layer Edge.Cuts) (width 0.1))
 (gr_line (start 263.398 153.416) (end 57.658 153.416) (layer Edge.Cuts) (width 0.1))
 (segment (start 166.878 26.136) (end 164.618 23.876) (width 0.25) (layer F.Cu) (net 1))
 (segment (start 166.878 27.686) (end 166.878 26.136) (width 0.25) (layer F.Cu) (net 1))
 (segment (start 141.198 23.876) (end 138.938 26.136) (width 0.25) (layer F.Cu) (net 1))
 (segment (start 164.618 23.876) (end 141.198 23.876) (width 0.25) (layer F.Cu) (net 1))
 (segment (start 128.778 27.686) (end 128.778 25.146) (width 0.25) (layer F.Cu) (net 1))
 (segment (start 128.778 25.146) (end 130.048 23.876) (width 0.25) (layer F.Cu) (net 1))
 (segment (start 138.938 26.136) (end 138.938 27.686) (width 0.25) (layer F.Cu) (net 1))
 (segment (start 136.678 23.876) (end 138.938 26.136) (width 0.25) (layer F.Cu) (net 1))
 (segment (start 130.048 23.876) (end 136.678 23.876) (width 0.25) (layer F.Cu) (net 1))
 (segment (start 128.778 27.686) (end 128.778 63.246) (width 0.25) (layer F.Cu) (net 1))
 (segment (start 129.794 64.262) (end 129.794 70.866) (width 0.25) (layer F.Cu) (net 1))
 (segment (start 128.778 63.246) (end 129.794 64.262) (width 0.25) (layer F.Cu) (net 1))
 (segment (start 217.678 96.266) (end 217.678 89.916) (width 0.25) (layer F.Cu) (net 1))
 (segment (start 199.898 114.046) (end 217.678 96.266) (width 0.25) (layer F.Cu) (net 1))
 (segment (start 217.678 89.916) (end 224.028 89.916) (width 0.25) (layer F.Cu) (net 1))
 (segment (start 199.898 70.866) (end 212.598 83.566) (width 0.25) (layer B.Cu) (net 37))
 (segment (start 197.358 70.866) (end 199.898 70.866) (width 0.25) (layer B.Cu) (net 37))
 (segment (start 217.678 86.601) (end 217.678 87.376) (width 0.25) (layer B.Cu) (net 37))
 (segment (start 214.643 83.566) (end 217.678 86.601) (width 0.25) (layer B.Cu) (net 37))
 (segment (start 212.598 83.566) (end 214.643 83.566) (width 0.25) (layer B.Cu) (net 37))
 (segment (start 217.678 87.376) (end 224.028 87.376) (width 0.25) (layer B.Cu) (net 37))
 (segment (start 208.788 83.566) (end 208.788 60.706) (width 0.25) (layer F.Cu) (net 4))
 (segment (start 208.788 60.706) (end 198.628 50.546) (width 0.25) (layer F.Cu) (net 4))
 (segment (start 164.338 29.236) (end 164.338 27.686) (width 0.25) (layer F.Cu) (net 4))
 (segment (start 185.648 50.546) (end 164.338 29.236) (width 0.25) (layer F.Cu) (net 4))
 (segment (start 198.628 50.546) (end 185.648 50.546) (width 0.25) (layer F.Cu) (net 4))
 (segment (start 161.798 27.686) (end 161.798 70.866) (width 0.25) (layer F.Cu) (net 63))
 (segment (start 159.258 27.686) (end 159.258 70.866) (width 0.25) (layer F.Cu) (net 62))
 (segment (start 156.718 29.236) (end 156.718 70.866) (width 0.25) (layer F.Cu) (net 61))
 (segment (start 156.718 27.686) (end 156.718 29.236) (width 0.25) (layer F.Cu) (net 61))
 (segment (start 154.178 27.686) (end 154.178 70.866) (width 0.25) (layer F.Cu) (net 60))
 (segment (start 137.414 70.866) (end 137.414 59.69) (width 0.25) (layer F.Cu) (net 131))
 (segment (start 141.478 55.626) (end 141.478 27.686) (width 0.25) (layer F.Cu) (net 131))
 (segment (start 137.414 59.69) (end 141.478 55.626) (width 0.25) (layer F.Cu) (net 131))
 (segment (start 134.874 69.6) (end 135.128 69.346) (width 0.25) (layer F.Cu) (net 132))
 (segment (start 134.874 70.866) (end 134.874 69.6) (width 0.25) (layer F.Cu) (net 132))
 (segment (start 135.128 69.346) (end 135.128 58.166) (width 0.25) (layer F.Cu) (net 132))
 (segment (start 136.398 56.896) (end 136.398 27.686) (width 0.25) (layer F.Cu) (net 132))
 (segment (start 135.128 58.166) (end 136.398 56.896) (width 0.25) (layer F.Cu) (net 132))
 (segment (start 198.221599 92.862401) (end 197.358 93.726) (width 0.25) (layer F.Cu) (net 20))
 (segment (start 198.546601 92.537399) (end 198.221599 92.862401) (width 0.25) (layer F.Cu) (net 20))
 (segment (start 207.599399 92.537399) (end 198.546601 92.537399) (width 0.25) (layer F.Cu) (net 20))
 (segment (start 208.788 93.726) (end 207.599399 92.537399) (width 0.25) (layer F.Cu) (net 20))
 (segment (start 211.798001 92.926001) (end 212.598 93.726) (width 0.25) (layer F.Cu) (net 3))
 (segment (start 207.662999 88.790999) (end 211.798001 92.926001) (width 0.25) (layer F.Cu) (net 3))
 (segment (start 207.662999 81.951869) (end 207.662999 88.790999) (width 0.25) (layer F.Cu) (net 3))
 (segment (start 198.546601 74.594601) (end 200.305731 74.594601) (width 0.25) (layer F.Cu) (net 3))
 (segment (start 200.305731 74.594601) (end 207.662999 81.951869) (width 0.25) (layer F.Cu) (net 3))
 (segment (start 197.358 73.406) (end 198.546601 74.594601) (width 0.25) (layer F.Cu) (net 3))
 (segment (start 216.678 88.646) (end 217.678 88.646) (width 0.25) (layer F.Cu) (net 3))
 (segment (start 216.54663 88.646) (end 216.678 88.646) (width 0.25) (layer F.Cu) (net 3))
 (segment (start 212.598 92.59463) (end 216.54663 88.646) (width 0.25) (layer F.Cu) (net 3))
 (segment (start 212.598 93.726) (end 212.598 92.59463) (width 0.25) (layer F.Cu) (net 3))
 (segment (start 217.678 88.646) (end 224.028 88.646) (width 0.25) (layer F.Cu) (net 3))
 (segment (start 65.02299 55.88101) (end 66.548 54.356) (width 0.25) (layer F.Cu) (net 72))
 (segment (start 65.02299 85.007758) (end 65.02299 55.88101) (width 0.25) (layer F.Cu) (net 72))
 (segment (start 92.89299 105.23601) (end 85.251242 105.23601) (width 0.25) (layer F.Cu) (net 72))
 (segment (start 93.218 104.911) (end 92.89299 105.23601) (width 0.25) (layer F.Cu) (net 72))
 (segment (start 85.251242 105.23601) (end 65.02299 85.007758) (width 0.25) (layer F.Cu) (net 72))
 (segment (start 93.218 103.886) (end 93.218 104.911) (width 0.25) (layer F.Cu) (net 72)))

